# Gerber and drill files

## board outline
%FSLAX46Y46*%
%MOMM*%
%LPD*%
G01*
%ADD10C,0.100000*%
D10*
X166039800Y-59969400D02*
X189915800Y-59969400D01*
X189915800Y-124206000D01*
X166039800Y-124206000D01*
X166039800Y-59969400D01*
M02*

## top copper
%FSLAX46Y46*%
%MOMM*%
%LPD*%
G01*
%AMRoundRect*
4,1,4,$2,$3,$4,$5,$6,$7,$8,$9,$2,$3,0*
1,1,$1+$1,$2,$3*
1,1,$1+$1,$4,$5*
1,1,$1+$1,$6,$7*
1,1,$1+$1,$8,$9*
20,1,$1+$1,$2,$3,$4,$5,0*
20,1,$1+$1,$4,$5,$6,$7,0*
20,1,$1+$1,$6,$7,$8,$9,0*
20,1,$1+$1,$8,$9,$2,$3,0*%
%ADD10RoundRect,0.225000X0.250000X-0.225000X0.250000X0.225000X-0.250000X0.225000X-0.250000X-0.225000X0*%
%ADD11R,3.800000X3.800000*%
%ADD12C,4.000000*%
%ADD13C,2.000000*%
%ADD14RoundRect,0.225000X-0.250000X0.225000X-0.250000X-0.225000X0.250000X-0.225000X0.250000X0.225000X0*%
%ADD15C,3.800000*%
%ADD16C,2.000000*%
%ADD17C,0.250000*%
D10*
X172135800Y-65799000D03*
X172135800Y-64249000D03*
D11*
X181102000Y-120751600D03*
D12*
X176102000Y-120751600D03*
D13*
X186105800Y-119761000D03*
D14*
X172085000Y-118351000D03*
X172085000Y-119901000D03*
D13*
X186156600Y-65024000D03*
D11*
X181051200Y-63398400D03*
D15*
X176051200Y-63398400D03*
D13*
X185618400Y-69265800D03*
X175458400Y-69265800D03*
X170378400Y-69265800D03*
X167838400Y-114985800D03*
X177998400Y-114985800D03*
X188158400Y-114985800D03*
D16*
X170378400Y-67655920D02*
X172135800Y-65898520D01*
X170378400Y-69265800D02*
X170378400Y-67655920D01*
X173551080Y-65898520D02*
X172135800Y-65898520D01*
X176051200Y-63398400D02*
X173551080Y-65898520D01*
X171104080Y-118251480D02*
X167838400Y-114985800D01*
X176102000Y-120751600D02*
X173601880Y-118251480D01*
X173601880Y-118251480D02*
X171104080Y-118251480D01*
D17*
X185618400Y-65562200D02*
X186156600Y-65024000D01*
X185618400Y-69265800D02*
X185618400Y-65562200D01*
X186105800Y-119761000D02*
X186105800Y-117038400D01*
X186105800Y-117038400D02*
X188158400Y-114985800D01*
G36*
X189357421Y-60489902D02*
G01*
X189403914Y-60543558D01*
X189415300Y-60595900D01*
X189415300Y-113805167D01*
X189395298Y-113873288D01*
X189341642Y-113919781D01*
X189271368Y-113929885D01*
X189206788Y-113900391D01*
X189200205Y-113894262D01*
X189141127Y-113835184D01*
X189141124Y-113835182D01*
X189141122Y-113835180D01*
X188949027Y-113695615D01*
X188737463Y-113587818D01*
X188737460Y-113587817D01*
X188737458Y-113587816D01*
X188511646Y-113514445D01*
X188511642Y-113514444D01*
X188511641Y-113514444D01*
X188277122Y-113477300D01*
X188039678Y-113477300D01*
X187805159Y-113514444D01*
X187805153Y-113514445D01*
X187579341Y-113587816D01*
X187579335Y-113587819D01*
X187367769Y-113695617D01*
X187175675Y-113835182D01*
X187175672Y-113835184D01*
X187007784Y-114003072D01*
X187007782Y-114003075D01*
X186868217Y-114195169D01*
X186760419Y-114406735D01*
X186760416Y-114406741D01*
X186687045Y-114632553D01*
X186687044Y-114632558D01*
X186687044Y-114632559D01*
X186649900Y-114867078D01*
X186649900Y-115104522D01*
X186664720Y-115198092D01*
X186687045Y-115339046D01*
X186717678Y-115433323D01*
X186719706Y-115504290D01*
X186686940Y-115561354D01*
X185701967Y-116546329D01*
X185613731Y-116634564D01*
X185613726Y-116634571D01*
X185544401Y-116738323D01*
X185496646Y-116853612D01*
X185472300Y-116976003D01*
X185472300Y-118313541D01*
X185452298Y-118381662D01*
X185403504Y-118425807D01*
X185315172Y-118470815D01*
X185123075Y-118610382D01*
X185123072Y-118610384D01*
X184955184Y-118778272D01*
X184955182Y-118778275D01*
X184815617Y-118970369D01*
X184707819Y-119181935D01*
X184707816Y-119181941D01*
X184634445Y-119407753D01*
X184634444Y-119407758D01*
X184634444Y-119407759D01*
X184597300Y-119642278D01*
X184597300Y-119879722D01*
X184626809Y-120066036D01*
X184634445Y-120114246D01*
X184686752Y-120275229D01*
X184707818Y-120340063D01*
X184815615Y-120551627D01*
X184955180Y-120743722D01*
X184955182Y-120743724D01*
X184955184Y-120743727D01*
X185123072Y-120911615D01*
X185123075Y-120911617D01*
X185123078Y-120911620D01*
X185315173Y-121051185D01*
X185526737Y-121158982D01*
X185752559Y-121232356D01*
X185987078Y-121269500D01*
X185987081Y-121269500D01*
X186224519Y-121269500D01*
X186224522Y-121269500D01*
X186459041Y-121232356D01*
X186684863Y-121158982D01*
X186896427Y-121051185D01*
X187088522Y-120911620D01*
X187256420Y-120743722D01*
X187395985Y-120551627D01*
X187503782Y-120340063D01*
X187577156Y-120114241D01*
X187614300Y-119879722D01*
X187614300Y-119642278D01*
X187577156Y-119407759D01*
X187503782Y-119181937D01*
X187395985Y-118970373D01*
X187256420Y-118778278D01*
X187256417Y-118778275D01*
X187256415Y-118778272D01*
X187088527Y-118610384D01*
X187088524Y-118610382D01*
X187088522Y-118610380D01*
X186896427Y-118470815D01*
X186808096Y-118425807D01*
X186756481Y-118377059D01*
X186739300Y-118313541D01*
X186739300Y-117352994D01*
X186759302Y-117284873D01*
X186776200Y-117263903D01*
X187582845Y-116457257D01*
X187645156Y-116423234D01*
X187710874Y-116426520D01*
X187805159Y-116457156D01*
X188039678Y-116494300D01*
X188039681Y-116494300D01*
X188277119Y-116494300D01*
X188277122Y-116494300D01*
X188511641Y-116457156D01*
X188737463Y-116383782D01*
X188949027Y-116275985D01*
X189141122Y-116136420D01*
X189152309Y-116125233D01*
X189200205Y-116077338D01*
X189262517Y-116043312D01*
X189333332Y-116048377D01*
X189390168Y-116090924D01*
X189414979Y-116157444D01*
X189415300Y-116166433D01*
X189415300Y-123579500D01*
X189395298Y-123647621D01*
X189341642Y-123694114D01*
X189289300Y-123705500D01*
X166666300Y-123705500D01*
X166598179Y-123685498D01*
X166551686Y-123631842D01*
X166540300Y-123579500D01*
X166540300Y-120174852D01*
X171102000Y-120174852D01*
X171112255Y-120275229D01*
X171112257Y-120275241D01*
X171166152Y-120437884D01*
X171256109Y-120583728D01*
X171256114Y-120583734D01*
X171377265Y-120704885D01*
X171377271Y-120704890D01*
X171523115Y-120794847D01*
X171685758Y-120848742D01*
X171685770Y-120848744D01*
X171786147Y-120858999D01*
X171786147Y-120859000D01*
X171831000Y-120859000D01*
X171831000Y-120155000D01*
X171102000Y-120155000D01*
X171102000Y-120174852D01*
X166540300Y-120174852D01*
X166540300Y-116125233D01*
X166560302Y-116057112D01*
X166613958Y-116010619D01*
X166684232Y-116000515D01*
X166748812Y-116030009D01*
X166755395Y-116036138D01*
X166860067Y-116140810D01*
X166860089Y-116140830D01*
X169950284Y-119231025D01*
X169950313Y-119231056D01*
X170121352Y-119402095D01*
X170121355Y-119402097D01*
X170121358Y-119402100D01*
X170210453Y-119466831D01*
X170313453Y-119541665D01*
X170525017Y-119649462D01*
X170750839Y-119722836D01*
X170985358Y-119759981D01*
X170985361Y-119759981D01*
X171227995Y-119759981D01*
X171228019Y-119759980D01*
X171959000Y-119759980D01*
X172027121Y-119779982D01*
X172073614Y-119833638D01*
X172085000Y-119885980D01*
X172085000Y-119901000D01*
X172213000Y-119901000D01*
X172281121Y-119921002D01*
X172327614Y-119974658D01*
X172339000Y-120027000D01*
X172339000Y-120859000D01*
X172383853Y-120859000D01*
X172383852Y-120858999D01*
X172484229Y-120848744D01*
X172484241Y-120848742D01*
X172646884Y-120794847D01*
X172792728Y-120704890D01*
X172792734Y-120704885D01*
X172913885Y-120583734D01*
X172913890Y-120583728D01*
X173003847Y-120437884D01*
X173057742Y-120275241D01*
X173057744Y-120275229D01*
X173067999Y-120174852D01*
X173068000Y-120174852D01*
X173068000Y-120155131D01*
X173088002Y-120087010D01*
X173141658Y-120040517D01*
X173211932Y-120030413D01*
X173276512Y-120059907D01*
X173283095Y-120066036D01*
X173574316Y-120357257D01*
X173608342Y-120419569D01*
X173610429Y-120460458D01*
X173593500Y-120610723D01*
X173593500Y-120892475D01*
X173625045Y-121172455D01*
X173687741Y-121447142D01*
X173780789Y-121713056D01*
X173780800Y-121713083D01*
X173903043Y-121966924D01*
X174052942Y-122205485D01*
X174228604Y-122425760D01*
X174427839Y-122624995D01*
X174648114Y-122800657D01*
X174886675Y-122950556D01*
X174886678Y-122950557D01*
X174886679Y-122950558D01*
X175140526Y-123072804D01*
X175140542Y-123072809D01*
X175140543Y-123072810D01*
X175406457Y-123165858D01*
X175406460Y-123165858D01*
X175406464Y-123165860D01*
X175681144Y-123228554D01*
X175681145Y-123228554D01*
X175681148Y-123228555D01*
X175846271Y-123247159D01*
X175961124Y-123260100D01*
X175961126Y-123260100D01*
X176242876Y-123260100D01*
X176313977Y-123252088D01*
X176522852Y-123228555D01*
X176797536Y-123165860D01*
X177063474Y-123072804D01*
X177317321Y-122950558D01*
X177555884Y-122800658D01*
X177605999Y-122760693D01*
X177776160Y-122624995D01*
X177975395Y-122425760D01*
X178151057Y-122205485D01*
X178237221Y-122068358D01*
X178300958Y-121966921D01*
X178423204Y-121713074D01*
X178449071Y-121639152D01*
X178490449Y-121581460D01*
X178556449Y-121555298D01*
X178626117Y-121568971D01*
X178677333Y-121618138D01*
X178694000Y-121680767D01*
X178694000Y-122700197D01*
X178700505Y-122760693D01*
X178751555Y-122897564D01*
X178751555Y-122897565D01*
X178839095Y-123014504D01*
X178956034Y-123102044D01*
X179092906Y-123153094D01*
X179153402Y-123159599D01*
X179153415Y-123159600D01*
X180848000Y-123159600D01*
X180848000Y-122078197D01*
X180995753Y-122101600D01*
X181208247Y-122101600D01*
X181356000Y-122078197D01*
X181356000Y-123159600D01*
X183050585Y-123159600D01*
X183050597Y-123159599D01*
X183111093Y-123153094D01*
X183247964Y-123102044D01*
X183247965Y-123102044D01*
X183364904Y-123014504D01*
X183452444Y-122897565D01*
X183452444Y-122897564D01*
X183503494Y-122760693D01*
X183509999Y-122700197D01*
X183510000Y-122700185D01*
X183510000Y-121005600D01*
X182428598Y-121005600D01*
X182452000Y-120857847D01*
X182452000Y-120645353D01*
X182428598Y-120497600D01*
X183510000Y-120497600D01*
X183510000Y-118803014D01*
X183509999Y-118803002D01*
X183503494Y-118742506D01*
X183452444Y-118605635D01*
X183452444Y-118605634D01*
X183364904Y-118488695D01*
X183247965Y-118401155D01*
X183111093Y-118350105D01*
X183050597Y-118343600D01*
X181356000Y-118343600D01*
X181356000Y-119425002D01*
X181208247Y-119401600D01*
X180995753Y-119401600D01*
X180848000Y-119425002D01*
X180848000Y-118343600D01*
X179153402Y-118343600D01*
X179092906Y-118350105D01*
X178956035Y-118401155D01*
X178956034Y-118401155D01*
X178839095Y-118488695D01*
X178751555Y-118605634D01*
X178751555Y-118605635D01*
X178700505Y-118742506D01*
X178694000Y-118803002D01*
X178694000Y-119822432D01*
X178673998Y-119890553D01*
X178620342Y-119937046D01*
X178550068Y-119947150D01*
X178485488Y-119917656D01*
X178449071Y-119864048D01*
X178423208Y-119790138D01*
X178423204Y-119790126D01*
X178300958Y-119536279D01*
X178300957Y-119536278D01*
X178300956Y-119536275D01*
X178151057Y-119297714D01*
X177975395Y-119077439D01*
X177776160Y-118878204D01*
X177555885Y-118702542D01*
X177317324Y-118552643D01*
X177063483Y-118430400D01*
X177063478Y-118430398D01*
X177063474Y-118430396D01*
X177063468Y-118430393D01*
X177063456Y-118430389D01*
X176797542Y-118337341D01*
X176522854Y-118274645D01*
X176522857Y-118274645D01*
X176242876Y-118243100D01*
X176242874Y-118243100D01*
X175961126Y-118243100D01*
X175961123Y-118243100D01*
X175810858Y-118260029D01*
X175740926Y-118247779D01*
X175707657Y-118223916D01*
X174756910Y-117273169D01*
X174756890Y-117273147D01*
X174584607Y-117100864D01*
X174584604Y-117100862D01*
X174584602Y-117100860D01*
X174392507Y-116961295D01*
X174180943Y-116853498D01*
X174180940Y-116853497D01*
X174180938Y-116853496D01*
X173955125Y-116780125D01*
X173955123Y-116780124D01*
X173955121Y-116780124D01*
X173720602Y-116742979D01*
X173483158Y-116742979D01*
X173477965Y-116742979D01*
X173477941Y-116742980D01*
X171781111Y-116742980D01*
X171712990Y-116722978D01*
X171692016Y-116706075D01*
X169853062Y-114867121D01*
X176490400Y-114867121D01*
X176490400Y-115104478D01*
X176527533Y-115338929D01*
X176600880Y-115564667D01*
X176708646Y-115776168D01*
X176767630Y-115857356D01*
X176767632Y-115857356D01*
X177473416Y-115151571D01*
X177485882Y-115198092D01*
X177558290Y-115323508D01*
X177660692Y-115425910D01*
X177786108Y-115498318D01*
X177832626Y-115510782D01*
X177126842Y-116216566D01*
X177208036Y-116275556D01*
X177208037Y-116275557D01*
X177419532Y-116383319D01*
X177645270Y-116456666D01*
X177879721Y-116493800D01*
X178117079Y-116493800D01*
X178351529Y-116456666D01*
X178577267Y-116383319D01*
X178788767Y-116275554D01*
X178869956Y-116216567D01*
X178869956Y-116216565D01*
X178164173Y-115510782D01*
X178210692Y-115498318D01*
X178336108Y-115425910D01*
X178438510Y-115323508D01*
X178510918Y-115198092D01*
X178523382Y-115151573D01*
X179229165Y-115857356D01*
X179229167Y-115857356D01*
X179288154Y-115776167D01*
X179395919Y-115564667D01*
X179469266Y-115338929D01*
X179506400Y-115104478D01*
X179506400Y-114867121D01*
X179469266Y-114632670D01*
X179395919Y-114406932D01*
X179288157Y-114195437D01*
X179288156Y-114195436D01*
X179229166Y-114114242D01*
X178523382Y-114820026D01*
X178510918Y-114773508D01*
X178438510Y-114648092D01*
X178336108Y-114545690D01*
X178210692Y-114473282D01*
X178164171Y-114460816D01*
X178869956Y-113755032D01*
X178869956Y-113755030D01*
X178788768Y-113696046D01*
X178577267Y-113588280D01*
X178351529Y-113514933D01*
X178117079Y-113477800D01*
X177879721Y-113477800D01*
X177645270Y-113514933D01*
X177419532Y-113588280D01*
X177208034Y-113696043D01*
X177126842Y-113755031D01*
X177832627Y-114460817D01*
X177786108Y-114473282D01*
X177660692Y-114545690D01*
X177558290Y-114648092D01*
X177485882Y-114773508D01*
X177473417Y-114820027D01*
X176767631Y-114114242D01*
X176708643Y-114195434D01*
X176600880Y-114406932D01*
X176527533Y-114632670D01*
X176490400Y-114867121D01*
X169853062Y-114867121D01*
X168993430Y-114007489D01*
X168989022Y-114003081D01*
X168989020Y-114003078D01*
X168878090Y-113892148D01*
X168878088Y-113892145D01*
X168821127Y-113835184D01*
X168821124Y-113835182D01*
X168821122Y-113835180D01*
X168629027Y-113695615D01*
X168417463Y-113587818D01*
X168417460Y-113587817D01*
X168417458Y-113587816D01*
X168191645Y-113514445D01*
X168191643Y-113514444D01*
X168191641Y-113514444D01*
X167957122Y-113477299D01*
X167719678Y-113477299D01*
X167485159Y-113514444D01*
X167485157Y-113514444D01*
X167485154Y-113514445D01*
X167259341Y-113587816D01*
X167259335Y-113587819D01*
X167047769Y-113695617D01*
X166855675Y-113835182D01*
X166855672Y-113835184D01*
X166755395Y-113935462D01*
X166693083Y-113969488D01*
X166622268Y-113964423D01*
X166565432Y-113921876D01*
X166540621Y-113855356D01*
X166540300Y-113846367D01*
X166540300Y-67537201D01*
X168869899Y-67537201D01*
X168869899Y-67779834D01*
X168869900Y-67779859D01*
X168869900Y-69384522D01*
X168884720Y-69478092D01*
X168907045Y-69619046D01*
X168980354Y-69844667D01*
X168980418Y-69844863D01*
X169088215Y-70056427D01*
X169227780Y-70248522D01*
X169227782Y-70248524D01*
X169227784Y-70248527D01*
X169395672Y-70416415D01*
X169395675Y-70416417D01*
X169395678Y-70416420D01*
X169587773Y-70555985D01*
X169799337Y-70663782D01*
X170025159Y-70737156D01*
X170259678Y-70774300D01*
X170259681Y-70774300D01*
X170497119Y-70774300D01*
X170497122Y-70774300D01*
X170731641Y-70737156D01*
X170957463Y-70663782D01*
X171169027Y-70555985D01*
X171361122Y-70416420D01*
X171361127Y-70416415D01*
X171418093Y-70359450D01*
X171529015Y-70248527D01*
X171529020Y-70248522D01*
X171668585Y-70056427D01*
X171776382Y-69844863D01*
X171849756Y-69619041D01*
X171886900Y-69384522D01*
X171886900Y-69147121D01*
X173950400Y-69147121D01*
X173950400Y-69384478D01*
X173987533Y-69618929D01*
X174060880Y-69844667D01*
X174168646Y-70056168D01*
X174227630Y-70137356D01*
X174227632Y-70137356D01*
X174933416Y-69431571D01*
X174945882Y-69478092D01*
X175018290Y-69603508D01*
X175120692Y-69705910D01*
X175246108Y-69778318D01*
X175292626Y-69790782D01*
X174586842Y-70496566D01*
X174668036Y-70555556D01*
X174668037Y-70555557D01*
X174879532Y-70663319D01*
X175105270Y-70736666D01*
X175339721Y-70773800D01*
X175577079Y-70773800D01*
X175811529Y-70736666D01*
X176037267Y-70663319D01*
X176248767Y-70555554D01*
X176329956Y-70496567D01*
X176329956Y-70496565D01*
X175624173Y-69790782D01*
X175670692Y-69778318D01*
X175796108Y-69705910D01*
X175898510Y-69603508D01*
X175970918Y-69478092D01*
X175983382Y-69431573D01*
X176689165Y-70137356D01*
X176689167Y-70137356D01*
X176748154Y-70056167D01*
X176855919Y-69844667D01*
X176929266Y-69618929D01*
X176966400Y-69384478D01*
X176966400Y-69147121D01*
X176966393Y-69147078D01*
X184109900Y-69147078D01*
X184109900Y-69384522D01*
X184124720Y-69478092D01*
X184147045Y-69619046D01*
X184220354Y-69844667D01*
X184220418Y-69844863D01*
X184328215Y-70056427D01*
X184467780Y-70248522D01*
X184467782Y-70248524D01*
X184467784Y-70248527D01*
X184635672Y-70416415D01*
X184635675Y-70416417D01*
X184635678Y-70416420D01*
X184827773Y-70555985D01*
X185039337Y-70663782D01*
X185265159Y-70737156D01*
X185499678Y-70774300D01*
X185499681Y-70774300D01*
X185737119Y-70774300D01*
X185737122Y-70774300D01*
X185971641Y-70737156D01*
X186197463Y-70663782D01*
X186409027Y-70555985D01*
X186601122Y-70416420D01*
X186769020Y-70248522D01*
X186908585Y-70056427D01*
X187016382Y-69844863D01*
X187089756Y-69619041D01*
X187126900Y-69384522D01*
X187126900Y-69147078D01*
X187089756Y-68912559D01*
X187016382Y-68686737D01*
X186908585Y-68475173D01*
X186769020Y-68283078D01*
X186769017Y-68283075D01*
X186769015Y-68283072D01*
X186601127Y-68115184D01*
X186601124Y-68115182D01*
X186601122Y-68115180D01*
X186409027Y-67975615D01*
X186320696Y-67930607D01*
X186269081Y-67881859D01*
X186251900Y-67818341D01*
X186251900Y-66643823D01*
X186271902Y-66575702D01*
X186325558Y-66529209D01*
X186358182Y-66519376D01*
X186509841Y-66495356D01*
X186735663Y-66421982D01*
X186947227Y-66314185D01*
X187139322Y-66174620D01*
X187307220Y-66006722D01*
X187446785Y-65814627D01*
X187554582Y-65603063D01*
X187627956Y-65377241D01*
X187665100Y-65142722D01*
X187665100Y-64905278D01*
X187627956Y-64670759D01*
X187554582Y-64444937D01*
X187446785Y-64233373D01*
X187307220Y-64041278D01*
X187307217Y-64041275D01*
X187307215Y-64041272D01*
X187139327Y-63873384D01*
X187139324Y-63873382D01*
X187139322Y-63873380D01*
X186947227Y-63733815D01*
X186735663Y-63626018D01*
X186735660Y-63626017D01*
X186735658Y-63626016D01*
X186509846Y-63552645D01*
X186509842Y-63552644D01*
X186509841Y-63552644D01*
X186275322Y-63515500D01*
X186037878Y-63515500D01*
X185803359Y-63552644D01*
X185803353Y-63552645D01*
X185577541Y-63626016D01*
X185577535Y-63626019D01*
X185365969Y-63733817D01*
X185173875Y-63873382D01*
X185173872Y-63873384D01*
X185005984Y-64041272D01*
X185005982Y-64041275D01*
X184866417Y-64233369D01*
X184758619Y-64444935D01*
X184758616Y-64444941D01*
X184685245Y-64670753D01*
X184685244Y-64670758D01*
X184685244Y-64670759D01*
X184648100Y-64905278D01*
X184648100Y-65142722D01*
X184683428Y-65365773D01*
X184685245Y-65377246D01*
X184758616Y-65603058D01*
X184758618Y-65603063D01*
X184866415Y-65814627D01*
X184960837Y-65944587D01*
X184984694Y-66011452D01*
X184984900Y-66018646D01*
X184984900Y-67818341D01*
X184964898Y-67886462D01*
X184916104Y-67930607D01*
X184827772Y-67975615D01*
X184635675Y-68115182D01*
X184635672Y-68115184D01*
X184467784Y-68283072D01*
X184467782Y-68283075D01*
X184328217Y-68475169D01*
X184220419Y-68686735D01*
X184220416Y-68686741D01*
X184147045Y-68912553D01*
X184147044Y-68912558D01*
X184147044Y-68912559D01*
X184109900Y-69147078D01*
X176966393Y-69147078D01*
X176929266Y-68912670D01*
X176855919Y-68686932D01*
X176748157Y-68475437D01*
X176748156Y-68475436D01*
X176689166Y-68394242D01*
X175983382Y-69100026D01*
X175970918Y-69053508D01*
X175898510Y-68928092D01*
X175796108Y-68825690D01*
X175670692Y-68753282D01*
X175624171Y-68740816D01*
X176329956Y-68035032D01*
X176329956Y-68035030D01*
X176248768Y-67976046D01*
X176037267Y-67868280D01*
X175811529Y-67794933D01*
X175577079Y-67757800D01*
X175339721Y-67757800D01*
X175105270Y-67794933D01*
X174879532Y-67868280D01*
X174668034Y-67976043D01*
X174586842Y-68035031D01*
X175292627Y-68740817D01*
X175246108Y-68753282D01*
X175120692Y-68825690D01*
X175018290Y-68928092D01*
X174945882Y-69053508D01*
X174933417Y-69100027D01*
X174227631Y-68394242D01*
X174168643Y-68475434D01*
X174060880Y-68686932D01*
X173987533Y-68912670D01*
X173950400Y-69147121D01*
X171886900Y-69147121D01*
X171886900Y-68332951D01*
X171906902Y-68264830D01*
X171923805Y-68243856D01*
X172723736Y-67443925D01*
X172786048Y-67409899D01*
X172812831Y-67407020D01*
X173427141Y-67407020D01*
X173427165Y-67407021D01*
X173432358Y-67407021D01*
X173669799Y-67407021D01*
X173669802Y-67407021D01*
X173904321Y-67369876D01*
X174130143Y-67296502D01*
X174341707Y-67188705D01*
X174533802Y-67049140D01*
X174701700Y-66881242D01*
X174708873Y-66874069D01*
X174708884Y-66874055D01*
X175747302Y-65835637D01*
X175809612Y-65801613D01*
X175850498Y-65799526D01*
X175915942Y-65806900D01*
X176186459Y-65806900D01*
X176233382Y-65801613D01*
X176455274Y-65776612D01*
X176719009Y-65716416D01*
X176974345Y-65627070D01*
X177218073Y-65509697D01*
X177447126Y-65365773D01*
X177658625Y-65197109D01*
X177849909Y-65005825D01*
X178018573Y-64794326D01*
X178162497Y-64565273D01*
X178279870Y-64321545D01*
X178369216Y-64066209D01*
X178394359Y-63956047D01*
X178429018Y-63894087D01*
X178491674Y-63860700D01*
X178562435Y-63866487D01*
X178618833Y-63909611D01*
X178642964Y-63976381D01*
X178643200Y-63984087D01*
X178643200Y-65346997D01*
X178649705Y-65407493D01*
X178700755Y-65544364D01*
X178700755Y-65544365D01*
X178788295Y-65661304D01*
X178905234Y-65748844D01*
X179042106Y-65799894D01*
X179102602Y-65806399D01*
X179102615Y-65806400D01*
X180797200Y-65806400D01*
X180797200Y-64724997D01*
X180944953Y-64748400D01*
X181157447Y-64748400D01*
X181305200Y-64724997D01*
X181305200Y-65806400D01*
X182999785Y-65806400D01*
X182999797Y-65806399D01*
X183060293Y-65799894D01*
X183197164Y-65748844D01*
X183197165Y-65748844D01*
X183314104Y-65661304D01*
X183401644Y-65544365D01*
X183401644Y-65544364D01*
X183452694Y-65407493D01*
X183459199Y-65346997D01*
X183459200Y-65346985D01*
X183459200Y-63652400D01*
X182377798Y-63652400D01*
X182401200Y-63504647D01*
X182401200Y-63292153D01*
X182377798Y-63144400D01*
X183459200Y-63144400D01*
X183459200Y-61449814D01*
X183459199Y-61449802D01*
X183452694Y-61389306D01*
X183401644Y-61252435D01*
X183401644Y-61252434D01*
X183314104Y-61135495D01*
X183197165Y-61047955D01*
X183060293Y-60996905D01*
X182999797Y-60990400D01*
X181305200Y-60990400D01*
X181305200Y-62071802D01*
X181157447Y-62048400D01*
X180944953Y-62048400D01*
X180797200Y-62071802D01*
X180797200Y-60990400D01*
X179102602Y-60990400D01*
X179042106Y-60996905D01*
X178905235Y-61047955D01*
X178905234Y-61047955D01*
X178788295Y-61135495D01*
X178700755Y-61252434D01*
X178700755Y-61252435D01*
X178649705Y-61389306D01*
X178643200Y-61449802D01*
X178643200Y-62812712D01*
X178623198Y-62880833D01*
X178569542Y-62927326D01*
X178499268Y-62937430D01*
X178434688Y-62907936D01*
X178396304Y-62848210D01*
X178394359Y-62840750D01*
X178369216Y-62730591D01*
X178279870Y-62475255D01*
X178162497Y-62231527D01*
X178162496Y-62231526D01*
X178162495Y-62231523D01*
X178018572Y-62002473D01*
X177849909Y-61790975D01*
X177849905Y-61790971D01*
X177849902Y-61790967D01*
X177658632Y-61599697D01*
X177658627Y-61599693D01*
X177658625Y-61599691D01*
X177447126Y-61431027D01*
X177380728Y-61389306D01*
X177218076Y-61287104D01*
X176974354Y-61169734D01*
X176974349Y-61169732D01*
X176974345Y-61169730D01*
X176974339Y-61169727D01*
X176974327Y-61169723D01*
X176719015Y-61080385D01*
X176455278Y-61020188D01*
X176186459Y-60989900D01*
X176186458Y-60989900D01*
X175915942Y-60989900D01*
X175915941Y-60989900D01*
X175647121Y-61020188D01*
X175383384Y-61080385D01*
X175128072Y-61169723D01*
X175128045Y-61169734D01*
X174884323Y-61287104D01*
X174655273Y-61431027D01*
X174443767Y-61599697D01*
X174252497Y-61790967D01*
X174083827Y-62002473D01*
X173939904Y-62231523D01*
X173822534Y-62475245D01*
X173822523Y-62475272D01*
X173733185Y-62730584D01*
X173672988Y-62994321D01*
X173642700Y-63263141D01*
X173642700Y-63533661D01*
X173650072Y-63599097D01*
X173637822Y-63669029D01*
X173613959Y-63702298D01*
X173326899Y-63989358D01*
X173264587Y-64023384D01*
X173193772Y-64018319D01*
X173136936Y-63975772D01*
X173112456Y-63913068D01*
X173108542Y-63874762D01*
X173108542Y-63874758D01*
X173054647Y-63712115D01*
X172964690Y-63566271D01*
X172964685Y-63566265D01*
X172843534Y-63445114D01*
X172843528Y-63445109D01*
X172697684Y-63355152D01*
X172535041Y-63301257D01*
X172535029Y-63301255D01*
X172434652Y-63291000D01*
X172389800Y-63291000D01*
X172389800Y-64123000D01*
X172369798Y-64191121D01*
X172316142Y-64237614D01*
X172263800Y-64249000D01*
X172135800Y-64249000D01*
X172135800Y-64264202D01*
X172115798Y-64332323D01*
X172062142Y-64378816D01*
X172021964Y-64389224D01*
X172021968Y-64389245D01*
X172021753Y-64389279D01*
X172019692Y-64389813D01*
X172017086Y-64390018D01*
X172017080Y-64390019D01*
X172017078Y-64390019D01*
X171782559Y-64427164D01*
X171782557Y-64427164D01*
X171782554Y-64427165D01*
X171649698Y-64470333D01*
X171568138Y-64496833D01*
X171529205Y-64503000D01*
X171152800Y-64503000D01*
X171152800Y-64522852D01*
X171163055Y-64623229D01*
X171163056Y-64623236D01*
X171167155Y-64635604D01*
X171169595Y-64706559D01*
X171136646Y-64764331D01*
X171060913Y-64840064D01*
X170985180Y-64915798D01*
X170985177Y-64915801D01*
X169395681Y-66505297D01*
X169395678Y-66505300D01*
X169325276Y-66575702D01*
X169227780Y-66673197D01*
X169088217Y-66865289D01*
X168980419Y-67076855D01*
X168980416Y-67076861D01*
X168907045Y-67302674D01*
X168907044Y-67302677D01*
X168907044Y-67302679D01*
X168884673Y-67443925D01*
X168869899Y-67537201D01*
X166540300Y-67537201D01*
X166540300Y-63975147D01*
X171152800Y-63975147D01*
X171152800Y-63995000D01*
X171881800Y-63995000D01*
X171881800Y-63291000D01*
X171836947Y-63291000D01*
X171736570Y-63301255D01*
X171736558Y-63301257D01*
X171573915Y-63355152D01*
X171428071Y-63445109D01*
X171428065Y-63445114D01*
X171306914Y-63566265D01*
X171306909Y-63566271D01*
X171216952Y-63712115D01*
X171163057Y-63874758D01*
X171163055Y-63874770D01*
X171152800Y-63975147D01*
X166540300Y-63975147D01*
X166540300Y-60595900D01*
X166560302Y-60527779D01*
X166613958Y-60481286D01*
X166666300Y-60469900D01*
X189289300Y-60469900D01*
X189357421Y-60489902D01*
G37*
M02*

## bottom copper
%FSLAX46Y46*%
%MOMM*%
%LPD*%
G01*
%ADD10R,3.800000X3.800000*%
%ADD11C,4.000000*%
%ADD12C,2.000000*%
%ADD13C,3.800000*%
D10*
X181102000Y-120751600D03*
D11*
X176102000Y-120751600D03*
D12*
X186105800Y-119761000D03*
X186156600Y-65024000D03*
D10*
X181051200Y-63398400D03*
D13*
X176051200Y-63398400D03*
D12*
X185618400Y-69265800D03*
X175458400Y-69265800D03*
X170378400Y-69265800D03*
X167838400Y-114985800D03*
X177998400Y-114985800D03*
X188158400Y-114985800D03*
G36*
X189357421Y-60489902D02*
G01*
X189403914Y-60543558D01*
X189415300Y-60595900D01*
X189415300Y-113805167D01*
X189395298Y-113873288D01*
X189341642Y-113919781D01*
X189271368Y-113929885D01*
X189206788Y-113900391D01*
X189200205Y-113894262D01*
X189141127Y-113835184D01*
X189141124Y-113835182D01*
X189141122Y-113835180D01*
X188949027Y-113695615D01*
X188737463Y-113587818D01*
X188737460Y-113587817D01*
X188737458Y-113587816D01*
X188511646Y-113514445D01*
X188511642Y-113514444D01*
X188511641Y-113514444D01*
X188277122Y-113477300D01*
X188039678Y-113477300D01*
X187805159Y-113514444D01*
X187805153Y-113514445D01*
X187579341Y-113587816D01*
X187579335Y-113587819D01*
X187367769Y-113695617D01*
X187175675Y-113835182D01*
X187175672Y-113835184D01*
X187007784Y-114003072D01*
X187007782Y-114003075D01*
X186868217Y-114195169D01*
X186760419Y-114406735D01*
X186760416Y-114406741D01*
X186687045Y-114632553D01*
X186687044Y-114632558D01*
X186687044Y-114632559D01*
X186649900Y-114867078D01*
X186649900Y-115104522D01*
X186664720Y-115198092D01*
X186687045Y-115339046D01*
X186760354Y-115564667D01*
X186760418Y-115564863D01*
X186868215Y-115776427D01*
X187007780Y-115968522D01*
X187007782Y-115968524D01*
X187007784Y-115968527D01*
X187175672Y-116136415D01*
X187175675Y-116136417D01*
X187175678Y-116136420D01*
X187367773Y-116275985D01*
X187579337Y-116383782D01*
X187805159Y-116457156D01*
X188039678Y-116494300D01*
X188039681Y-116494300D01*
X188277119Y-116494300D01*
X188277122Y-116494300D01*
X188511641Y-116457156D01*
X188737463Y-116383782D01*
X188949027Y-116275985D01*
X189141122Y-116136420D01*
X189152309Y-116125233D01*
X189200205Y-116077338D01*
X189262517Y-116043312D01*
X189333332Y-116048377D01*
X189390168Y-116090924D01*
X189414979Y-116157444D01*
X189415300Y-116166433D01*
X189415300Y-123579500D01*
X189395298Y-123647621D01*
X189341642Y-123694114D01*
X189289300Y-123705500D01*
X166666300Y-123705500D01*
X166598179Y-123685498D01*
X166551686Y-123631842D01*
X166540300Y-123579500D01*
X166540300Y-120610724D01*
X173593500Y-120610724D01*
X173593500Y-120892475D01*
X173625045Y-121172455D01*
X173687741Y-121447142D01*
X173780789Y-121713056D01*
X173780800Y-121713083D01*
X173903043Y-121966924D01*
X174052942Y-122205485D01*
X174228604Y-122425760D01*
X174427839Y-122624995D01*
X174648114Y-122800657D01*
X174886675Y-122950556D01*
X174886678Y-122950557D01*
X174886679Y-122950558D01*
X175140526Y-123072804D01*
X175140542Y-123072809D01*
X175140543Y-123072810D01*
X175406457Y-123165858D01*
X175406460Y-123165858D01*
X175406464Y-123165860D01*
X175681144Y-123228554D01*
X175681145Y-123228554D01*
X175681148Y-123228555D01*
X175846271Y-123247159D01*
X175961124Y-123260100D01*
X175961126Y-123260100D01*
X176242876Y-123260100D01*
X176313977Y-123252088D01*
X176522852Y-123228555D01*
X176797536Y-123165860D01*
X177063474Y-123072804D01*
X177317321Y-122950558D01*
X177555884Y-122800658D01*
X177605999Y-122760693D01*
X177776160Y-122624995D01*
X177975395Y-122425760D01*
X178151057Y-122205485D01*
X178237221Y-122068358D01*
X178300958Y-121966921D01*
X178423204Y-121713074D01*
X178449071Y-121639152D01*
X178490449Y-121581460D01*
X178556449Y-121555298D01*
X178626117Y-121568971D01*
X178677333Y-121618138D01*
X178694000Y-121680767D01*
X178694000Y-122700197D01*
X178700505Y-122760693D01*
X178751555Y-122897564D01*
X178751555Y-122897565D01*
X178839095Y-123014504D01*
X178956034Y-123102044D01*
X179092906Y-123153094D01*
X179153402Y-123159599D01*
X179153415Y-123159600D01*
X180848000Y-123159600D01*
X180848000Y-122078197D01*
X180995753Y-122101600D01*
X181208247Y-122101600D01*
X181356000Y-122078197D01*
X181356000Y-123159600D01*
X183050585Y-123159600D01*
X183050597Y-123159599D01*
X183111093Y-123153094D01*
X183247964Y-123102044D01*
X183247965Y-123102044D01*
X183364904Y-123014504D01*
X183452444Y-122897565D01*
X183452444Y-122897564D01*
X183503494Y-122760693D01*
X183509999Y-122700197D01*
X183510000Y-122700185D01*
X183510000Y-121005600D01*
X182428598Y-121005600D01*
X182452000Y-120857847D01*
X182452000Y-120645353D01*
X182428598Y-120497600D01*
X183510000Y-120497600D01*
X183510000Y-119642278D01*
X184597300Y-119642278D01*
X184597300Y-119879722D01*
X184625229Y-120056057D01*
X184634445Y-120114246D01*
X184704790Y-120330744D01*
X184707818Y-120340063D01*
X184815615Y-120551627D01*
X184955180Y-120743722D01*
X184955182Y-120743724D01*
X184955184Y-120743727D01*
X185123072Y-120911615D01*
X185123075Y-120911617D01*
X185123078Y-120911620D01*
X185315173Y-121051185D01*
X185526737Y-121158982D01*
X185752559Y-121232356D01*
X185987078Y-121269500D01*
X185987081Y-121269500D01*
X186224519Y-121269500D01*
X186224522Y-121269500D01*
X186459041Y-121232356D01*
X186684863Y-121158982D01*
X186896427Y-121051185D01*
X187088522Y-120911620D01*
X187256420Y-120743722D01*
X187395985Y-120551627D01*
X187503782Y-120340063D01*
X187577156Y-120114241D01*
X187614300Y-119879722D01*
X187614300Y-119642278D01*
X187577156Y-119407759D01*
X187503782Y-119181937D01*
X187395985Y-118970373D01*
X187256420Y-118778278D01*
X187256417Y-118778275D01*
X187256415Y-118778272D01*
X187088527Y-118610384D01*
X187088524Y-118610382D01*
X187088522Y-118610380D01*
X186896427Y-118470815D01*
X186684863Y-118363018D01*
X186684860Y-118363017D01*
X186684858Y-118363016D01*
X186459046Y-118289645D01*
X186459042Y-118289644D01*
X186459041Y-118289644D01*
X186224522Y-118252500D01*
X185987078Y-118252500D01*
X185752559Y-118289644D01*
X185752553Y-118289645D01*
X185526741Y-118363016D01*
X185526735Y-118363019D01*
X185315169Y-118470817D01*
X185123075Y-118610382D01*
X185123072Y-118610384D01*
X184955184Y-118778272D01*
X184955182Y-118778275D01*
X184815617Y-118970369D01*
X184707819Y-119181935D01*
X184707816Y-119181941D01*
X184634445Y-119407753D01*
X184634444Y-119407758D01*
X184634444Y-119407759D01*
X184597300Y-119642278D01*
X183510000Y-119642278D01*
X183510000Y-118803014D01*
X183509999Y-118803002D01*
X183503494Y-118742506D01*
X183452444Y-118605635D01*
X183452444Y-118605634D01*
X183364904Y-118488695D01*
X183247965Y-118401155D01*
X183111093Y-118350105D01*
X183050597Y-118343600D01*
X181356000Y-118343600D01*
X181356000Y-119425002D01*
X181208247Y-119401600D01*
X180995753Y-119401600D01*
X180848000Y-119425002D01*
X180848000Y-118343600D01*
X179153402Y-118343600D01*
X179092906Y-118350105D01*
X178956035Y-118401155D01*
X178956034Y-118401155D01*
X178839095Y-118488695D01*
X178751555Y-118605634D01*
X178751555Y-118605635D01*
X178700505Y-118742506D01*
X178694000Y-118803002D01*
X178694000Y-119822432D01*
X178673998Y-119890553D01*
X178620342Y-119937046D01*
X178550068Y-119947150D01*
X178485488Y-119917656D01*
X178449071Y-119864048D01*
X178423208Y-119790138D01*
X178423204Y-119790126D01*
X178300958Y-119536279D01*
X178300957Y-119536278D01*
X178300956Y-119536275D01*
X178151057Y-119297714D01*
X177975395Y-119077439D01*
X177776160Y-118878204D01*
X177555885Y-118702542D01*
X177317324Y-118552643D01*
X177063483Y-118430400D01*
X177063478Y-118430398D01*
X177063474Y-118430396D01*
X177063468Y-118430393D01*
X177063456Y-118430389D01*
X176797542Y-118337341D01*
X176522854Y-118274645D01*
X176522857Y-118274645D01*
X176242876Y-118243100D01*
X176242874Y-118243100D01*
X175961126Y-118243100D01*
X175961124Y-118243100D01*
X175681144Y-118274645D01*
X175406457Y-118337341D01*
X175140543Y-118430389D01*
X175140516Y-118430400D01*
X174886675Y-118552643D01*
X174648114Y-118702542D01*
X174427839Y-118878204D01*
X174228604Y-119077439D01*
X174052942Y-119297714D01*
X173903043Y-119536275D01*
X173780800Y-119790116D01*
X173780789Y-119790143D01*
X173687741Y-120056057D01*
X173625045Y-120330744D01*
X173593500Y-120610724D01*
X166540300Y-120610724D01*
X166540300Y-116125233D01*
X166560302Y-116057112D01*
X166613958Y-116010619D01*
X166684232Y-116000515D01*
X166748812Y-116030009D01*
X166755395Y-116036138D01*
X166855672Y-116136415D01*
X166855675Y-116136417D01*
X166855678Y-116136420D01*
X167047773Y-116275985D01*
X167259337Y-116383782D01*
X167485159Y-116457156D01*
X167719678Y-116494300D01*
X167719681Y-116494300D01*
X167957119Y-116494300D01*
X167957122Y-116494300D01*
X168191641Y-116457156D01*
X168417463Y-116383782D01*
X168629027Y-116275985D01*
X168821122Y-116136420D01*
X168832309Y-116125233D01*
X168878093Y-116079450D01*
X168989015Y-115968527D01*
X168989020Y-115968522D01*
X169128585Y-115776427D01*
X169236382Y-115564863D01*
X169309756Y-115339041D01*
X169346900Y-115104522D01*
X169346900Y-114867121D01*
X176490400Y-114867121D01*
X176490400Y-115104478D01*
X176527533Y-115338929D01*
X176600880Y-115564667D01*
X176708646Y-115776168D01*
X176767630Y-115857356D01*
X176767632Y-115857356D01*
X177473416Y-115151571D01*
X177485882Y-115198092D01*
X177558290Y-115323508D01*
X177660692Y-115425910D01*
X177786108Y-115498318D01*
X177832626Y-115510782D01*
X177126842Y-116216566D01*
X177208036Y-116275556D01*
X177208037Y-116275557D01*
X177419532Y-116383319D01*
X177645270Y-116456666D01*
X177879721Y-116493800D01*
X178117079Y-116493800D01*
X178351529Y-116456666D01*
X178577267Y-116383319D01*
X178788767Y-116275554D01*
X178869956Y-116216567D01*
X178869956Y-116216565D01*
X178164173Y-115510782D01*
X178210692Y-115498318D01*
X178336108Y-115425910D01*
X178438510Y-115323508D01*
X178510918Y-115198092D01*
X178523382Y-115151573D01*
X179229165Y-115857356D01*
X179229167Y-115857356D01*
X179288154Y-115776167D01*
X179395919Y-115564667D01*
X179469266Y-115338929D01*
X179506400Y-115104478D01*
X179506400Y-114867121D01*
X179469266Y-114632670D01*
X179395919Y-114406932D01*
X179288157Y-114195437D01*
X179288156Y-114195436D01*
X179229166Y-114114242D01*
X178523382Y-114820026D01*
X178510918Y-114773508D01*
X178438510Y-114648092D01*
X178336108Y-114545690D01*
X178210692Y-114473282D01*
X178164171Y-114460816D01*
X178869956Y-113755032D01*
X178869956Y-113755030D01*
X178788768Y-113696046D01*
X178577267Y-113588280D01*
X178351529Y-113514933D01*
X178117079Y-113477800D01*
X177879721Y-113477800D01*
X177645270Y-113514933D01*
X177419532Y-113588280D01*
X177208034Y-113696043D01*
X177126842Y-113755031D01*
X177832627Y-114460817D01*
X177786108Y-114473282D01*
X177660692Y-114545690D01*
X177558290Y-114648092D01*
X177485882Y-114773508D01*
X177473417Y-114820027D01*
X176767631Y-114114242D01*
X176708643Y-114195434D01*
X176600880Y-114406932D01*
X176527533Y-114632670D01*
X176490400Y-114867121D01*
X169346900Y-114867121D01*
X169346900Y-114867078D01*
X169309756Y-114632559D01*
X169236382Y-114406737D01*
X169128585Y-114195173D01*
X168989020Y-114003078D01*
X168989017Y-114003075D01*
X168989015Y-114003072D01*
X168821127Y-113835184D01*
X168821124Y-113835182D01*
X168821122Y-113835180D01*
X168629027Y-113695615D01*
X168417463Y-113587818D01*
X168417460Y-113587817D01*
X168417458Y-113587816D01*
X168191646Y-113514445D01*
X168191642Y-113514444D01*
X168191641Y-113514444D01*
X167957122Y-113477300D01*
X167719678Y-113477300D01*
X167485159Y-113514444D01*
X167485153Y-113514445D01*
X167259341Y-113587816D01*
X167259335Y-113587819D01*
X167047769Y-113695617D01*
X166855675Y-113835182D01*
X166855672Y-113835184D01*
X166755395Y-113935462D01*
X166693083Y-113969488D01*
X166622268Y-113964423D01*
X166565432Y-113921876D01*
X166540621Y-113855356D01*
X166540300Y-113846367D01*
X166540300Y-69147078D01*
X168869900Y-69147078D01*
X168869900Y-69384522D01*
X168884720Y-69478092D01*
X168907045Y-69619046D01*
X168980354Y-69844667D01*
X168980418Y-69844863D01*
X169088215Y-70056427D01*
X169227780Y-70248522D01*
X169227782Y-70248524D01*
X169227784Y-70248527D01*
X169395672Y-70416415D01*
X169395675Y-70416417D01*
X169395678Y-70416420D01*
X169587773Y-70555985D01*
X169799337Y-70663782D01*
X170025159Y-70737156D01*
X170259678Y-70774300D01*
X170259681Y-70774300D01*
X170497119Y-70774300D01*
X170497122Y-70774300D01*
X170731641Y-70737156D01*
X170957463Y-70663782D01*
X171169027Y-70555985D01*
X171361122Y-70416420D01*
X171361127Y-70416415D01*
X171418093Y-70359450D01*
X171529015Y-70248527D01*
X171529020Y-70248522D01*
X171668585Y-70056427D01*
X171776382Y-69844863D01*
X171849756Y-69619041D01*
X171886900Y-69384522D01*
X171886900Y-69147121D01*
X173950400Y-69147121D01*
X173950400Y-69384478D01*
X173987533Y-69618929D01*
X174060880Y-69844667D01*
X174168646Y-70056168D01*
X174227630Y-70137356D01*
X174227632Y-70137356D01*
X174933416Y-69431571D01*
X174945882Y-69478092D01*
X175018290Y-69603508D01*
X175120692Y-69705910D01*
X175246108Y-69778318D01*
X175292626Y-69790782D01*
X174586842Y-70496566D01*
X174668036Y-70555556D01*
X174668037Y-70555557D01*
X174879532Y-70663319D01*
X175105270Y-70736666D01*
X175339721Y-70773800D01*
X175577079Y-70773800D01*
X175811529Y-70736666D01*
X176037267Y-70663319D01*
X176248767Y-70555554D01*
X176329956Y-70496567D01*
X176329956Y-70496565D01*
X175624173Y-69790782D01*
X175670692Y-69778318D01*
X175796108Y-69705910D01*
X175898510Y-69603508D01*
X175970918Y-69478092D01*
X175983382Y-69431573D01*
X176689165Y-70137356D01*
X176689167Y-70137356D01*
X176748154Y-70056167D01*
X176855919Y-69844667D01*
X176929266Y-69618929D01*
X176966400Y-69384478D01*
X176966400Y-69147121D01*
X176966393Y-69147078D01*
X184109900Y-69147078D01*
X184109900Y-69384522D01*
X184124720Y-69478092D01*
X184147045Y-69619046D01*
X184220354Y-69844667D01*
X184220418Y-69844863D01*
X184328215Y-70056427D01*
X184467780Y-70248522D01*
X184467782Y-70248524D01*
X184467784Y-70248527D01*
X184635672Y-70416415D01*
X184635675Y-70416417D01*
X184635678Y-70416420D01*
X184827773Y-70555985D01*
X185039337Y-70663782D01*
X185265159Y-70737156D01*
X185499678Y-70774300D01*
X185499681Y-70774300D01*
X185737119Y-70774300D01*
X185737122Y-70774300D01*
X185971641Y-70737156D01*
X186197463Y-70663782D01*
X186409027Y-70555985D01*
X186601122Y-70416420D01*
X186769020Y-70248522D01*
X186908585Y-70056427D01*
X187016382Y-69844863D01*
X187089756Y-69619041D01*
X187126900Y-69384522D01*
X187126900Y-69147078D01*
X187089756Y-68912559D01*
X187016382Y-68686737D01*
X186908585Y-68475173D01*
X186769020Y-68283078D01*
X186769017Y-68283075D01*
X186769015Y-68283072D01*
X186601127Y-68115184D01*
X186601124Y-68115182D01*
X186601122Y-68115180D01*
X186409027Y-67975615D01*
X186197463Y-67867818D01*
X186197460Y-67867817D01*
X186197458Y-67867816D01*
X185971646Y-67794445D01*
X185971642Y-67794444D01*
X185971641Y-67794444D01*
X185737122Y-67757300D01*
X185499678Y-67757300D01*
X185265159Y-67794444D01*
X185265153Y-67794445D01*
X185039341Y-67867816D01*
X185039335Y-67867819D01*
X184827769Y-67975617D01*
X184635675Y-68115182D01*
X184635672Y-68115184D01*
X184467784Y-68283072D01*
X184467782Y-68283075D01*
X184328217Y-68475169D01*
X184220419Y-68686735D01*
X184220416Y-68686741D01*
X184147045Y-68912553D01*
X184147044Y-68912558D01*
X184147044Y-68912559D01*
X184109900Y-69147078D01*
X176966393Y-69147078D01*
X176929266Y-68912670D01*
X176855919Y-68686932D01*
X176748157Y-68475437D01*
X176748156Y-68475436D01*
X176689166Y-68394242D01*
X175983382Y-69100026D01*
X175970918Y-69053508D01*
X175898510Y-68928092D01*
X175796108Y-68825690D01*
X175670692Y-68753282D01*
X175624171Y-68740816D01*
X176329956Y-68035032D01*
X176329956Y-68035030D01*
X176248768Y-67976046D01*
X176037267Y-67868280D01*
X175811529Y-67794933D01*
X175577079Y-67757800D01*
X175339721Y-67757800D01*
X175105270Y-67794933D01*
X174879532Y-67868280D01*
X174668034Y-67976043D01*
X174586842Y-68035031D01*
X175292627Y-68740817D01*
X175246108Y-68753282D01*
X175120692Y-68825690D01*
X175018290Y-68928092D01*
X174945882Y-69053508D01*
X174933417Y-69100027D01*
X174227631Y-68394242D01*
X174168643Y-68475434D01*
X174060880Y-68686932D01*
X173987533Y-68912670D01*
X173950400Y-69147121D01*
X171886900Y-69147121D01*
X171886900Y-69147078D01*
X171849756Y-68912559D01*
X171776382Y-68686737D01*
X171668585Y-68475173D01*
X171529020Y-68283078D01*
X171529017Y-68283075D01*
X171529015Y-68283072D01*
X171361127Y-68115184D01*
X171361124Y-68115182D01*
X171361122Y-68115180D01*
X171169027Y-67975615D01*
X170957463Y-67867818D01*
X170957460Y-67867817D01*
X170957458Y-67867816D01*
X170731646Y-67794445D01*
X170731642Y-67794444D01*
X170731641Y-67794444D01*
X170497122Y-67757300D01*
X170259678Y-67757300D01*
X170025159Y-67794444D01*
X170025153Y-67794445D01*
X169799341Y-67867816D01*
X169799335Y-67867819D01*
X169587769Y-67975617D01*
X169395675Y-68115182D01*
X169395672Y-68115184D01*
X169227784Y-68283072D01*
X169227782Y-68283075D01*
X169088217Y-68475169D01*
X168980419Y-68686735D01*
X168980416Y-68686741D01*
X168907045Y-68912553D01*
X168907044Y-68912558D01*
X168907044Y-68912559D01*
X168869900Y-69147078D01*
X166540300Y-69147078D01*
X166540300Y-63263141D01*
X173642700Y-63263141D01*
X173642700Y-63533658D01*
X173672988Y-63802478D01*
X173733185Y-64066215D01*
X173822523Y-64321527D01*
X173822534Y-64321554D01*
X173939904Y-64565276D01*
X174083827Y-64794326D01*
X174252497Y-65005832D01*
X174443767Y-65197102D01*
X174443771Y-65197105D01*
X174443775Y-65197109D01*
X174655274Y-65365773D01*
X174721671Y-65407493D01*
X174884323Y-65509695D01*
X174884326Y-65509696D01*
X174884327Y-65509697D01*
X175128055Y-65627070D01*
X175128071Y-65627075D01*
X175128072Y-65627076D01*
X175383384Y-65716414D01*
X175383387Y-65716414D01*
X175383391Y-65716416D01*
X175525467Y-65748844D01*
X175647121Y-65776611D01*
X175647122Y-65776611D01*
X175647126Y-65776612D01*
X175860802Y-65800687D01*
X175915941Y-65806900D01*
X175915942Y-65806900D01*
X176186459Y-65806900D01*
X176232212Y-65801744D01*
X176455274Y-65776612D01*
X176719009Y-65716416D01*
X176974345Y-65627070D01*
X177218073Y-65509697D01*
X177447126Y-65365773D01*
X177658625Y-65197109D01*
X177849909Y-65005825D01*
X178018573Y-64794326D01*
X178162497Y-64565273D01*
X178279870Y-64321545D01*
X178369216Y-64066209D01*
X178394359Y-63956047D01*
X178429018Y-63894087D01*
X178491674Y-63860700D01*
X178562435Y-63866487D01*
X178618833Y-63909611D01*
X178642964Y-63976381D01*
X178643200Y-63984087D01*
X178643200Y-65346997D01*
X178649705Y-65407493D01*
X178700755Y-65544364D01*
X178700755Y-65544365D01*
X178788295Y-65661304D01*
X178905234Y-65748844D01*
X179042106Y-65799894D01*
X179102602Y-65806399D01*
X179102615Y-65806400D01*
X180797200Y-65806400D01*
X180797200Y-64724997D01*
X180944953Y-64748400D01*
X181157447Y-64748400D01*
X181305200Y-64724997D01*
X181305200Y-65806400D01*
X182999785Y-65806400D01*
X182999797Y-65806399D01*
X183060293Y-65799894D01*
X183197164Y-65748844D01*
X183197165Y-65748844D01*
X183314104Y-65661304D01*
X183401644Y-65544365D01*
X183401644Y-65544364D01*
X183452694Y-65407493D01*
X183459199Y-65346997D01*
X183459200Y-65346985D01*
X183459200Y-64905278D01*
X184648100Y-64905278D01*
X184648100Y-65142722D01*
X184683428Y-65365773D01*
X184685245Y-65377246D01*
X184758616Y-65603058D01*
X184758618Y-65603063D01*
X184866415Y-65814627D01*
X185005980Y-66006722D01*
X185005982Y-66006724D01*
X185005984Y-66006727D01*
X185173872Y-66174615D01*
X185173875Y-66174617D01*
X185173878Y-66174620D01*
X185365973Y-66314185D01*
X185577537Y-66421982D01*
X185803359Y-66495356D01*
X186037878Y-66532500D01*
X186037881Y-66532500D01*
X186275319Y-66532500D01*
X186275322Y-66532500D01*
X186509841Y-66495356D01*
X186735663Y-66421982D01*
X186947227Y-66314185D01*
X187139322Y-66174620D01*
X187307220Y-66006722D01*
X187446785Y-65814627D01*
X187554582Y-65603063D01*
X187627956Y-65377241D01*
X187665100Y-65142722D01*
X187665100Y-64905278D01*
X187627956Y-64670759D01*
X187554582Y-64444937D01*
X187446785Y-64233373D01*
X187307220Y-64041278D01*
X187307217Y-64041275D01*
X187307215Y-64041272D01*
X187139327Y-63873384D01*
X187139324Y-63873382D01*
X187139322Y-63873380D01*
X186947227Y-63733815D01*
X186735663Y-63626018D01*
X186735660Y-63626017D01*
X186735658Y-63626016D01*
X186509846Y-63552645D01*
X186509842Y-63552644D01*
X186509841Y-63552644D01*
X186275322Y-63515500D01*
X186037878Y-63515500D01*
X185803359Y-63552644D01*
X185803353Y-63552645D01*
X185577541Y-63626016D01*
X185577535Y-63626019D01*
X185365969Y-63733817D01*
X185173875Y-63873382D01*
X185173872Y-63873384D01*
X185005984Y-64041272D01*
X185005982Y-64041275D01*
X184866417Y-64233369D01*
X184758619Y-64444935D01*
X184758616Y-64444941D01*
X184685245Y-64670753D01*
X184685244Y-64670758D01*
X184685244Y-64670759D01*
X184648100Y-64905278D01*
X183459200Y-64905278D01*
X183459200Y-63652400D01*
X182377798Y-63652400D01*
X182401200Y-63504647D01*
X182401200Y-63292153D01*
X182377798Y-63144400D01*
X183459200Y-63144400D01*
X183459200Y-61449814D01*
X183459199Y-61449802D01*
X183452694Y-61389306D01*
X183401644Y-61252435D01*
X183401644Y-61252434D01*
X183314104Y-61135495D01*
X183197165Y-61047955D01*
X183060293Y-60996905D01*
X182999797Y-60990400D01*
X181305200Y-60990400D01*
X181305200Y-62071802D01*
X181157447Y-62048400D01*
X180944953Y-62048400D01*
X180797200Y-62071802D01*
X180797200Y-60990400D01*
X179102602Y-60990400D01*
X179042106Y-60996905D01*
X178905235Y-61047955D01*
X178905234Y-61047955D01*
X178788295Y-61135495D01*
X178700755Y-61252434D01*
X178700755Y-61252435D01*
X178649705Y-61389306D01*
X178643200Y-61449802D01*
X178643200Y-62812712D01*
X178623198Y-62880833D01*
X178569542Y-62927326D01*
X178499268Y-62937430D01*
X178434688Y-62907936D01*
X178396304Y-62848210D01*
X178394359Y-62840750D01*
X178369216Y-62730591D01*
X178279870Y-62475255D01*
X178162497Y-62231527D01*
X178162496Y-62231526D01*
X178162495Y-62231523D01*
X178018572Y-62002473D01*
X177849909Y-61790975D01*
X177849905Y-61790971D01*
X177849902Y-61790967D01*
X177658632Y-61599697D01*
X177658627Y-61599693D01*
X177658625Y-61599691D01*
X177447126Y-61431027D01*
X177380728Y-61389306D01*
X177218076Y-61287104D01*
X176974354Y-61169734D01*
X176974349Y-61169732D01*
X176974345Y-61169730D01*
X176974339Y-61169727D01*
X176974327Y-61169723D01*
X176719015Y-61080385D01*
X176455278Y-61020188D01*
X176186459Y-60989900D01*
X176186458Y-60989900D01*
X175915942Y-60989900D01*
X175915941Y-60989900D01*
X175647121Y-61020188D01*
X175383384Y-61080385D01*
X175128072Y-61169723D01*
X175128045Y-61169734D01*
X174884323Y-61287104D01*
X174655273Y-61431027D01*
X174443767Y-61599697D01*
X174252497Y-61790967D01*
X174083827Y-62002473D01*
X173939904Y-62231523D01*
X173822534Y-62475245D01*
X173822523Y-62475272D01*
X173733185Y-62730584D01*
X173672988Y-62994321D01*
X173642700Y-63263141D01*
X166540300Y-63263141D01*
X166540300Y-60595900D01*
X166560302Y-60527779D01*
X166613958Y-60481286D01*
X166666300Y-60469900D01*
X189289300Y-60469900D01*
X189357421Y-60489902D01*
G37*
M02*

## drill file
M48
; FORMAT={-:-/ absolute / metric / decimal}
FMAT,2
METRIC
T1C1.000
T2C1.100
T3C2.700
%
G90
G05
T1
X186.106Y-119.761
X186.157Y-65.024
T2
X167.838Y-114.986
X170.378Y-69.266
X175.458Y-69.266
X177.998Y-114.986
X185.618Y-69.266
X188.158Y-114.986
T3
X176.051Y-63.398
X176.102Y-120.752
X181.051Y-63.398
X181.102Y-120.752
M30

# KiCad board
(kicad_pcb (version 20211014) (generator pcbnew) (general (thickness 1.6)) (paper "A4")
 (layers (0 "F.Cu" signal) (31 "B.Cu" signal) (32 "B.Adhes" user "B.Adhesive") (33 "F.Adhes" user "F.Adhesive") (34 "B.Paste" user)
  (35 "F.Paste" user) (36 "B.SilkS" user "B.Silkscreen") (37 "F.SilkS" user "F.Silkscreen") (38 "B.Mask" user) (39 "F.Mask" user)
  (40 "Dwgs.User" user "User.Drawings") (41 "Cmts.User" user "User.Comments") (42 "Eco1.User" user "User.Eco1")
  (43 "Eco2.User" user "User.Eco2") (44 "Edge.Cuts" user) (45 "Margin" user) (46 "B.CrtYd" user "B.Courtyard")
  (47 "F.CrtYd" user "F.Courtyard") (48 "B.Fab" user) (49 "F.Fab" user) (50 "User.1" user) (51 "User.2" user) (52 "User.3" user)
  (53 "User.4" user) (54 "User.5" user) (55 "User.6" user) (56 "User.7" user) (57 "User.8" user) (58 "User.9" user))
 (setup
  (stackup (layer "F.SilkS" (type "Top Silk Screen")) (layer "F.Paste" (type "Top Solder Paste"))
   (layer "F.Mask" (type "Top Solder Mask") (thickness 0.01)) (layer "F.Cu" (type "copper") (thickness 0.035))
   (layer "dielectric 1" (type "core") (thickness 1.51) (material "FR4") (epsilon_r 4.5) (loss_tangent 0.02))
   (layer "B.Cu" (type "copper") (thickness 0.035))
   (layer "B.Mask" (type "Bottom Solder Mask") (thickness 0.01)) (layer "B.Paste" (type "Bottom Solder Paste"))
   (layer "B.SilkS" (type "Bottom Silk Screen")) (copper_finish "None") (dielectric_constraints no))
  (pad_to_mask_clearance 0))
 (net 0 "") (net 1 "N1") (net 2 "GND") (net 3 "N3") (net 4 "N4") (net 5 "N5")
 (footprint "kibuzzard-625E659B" (layer "F.Cu") (at 170.2308 63.5254 90)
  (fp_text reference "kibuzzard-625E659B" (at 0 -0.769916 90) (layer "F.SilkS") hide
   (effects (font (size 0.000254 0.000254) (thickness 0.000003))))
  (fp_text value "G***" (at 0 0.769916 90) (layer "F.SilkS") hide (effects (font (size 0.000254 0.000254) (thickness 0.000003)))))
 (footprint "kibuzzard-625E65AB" (layer "F.Cu") (at 168.91 120.8278 90)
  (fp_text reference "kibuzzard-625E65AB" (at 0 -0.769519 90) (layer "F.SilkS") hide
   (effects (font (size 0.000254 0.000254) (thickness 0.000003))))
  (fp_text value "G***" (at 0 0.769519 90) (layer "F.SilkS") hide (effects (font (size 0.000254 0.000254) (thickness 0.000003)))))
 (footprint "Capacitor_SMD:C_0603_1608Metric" (layer "F.Cu") (at 172.1358 65.024 90)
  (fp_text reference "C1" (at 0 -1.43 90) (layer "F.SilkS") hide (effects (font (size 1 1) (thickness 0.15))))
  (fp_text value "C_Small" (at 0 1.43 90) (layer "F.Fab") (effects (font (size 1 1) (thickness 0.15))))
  (pad "1" smd roundrect (at -0.775 0 90) (size 0.9 0.95) (layers "F.Cu" "F.Paste" "F.Mask") (roundrect_rratio 0.25) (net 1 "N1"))
  (pad "2" smd roundrect (at 0.775 0 90) (size 0.9 0.95) (layers "F.Cu" "F.Paste" "F.Mask") (roundrect_rratio 0.25) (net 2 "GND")))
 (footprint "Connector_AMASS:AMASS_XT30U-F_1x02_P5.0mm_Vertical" (layer "F.Cu") (at 181.102 120.7516 180)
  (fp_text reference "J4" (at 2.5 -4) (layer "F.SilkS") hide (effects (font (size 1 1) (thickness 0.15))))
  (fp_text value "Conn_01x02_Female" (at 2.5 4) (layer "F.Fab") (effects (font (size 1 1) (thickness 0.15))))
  (pad "1" thru_hole rect (at 0 0 180) (size 3.8 3.8) (drill 2.7) (layers *.Cu *.Mask) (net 2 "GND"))
  (pad "2" thru_hole circle (at 5 0 180) (size 4 4) (drill 2.7) (layers *.Cu *.Mask) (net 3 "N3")))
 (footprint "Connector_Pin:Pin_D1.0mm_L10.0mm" (layer "F.Cu") (at 186.1058 119.761)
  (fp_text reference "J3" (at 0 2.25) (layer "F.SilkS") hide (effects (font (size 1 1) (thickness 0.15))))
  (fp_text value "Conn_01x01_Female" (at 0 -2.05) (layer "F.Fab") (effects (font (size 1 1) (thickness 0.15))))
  (pad "1" thru_hole circle (at 0 0) (size 2 2) (drill 1) (layers *.Cu *.Mask) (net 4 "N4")))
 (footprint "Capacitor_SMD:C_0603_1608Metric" (layer "F.Cu") (at 172.085 119.126 -90)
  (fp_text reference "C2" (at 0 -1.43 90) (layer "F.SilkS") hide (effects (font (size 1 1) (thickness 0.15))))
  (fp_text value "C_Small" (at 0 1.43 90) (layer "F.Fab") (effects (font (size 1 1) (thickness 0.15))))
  (pad "1" smd roundrect (at -0.775 0 270) (size 0.9 0.95) (layers "F.Cu" "F.Paste" "F.Mask") (roundrect_rratio 0.25) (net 3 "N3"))
  (pad "2" smd roundrect (at 0.775 0 270) (size 0.9 0.95) (layers "F.Cu" "F.Paste" "F.Mask") (roundrect_rratio 0.25) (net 2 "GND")))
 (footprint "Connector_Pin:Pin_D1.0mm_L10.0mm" (layer "F.Cu") (at 186.1566 65.024)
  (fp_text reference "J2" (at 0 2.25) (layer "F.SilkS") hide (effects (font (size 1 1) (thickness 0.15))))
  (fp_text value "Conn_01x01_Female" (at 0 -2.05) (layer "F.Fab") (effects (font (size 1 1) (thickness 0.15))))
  (pad "1" thru_hole circle (at 0 0) (size 2 2) (drill 1) (layers *.Cu *.Mask) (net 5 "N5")))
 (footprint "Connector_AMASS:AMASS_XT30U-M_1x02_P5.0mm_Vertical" (layer "F.Cu") (at 181.0512 63.3984 180)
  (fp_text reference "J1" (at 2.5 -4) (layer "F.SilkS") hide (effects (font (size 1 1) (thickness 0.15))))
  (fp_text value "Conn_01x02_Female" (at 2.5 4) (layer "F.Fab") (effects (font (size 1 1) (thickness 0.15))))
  (pad "1" thru_hole rect (at 0 0 180) (size 3.8 3.8) (drill 2.7) (layers *.Cu *.Mask) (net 2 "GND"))
  (pad "2" thru_hole circle (at 5 0 180) (size 3.8 3.8) (drill 2.7) (layers *.Cu *.Mask) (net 1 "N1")))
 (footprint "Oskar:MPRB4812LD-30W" (layer "F.Cu") (at 177.6984 92.1258 -90)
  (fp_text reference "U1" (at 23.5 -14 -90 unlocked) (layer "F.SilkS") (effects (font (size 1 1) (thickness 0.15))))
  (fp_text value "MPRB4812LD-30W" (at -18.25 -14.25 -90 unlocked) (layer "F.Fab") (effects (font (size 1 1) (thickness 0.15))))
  (pad "1" thru_hole circle (at -22.86 -7.92 270) (size 2 2) (drill 1.1) (layers *.Cu *.Mask) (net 5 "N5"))
  (pad "2" thru_hole circle (at -22.86 2.24 270) (size 2 2) (drill 1.1) (layers *.Cu *.Mask) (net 2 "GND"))
  (pad "3" thru_hole circle (at -22.86 7.32 270) (size 2 2) (drill 1.1) (layers *.Cu *.Mask) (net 1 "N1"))
  (pad "4" thru_hole circle (at 22.86 9.86 270) (size 2 2) (drill 1.1) (layers *.Cu *.Mask) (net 3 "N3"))
  (pad "5" thru_hole circle (at 22.86 -0.3 270) (size 2 2) (drill 1.1) (layers *.Cu *.Mask) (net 2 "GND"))
  (pad "6" thru_hole circle (at 22.86 -10.46 270) (size 2 2) (drill 1.1) (layers *.Cu *.Mask) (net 4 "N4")))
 (gr_rect (start 166.0398 59.9694) (end 189.9158 124.206) (layer "Edge.Cuts") (width 0.1) (fill none))
 (segment (start 170.3784 67.65592) (end 172.1358 65.89852) (width 2) (layer "F.Cu") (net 1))
 (segment (start 170.3784 69.2658) (end 170.3784 67.65592) (width 2) (layer "F.Cu") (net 1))
 (segment (start 173.55108 65.89852) (end 172.1358 65.89852) (width 2) (layer "F.Cu") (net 1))
 (segment (start 176.0512 63.3984) (end 173.55108 65.89852) (width 2) (layer "F.Cu") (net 1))
 (segment (start 171.10408 118.25148) (end 167.8384 114.9858) (width 2) (layer "F.Cu") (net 3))
 (segment (start 176.102 120.7516) (end 173.60188 118.25148) (width 2) (layer "F.Cu") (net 3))
 (segment (start 173.60188 118.25148) (end 171.10408 118.25148) (width 2) (layer "F.Cu") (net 3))
 (segment (start 185.6184 65.5622) (end 186.1566 65.024) (width 0.25) (layer "F.Cu") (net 5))
 (segment (start 185.6184 69.2658) (end 185.6184 65.5622) (width 0.25) (layer "F.Cu") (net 5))
 (segment (start 186.1058 119.761) (end 186.1058 117.0384) (width 0.25) (layer "F.Cu") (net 4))
 (segment (start 186.1058 117.0384) (end 188.1584 114.9858) (width 0.25) (layer "F.Cu") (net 4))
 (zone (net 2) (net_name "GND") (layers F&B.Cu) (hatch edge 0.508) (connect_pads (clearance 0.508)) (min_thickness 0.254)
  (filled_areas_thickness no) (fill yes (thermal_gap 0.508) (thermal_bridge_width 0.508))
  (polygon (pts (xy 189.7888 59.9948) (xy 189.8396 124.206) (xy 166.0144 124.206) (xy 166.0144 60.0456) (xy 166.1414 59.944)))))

